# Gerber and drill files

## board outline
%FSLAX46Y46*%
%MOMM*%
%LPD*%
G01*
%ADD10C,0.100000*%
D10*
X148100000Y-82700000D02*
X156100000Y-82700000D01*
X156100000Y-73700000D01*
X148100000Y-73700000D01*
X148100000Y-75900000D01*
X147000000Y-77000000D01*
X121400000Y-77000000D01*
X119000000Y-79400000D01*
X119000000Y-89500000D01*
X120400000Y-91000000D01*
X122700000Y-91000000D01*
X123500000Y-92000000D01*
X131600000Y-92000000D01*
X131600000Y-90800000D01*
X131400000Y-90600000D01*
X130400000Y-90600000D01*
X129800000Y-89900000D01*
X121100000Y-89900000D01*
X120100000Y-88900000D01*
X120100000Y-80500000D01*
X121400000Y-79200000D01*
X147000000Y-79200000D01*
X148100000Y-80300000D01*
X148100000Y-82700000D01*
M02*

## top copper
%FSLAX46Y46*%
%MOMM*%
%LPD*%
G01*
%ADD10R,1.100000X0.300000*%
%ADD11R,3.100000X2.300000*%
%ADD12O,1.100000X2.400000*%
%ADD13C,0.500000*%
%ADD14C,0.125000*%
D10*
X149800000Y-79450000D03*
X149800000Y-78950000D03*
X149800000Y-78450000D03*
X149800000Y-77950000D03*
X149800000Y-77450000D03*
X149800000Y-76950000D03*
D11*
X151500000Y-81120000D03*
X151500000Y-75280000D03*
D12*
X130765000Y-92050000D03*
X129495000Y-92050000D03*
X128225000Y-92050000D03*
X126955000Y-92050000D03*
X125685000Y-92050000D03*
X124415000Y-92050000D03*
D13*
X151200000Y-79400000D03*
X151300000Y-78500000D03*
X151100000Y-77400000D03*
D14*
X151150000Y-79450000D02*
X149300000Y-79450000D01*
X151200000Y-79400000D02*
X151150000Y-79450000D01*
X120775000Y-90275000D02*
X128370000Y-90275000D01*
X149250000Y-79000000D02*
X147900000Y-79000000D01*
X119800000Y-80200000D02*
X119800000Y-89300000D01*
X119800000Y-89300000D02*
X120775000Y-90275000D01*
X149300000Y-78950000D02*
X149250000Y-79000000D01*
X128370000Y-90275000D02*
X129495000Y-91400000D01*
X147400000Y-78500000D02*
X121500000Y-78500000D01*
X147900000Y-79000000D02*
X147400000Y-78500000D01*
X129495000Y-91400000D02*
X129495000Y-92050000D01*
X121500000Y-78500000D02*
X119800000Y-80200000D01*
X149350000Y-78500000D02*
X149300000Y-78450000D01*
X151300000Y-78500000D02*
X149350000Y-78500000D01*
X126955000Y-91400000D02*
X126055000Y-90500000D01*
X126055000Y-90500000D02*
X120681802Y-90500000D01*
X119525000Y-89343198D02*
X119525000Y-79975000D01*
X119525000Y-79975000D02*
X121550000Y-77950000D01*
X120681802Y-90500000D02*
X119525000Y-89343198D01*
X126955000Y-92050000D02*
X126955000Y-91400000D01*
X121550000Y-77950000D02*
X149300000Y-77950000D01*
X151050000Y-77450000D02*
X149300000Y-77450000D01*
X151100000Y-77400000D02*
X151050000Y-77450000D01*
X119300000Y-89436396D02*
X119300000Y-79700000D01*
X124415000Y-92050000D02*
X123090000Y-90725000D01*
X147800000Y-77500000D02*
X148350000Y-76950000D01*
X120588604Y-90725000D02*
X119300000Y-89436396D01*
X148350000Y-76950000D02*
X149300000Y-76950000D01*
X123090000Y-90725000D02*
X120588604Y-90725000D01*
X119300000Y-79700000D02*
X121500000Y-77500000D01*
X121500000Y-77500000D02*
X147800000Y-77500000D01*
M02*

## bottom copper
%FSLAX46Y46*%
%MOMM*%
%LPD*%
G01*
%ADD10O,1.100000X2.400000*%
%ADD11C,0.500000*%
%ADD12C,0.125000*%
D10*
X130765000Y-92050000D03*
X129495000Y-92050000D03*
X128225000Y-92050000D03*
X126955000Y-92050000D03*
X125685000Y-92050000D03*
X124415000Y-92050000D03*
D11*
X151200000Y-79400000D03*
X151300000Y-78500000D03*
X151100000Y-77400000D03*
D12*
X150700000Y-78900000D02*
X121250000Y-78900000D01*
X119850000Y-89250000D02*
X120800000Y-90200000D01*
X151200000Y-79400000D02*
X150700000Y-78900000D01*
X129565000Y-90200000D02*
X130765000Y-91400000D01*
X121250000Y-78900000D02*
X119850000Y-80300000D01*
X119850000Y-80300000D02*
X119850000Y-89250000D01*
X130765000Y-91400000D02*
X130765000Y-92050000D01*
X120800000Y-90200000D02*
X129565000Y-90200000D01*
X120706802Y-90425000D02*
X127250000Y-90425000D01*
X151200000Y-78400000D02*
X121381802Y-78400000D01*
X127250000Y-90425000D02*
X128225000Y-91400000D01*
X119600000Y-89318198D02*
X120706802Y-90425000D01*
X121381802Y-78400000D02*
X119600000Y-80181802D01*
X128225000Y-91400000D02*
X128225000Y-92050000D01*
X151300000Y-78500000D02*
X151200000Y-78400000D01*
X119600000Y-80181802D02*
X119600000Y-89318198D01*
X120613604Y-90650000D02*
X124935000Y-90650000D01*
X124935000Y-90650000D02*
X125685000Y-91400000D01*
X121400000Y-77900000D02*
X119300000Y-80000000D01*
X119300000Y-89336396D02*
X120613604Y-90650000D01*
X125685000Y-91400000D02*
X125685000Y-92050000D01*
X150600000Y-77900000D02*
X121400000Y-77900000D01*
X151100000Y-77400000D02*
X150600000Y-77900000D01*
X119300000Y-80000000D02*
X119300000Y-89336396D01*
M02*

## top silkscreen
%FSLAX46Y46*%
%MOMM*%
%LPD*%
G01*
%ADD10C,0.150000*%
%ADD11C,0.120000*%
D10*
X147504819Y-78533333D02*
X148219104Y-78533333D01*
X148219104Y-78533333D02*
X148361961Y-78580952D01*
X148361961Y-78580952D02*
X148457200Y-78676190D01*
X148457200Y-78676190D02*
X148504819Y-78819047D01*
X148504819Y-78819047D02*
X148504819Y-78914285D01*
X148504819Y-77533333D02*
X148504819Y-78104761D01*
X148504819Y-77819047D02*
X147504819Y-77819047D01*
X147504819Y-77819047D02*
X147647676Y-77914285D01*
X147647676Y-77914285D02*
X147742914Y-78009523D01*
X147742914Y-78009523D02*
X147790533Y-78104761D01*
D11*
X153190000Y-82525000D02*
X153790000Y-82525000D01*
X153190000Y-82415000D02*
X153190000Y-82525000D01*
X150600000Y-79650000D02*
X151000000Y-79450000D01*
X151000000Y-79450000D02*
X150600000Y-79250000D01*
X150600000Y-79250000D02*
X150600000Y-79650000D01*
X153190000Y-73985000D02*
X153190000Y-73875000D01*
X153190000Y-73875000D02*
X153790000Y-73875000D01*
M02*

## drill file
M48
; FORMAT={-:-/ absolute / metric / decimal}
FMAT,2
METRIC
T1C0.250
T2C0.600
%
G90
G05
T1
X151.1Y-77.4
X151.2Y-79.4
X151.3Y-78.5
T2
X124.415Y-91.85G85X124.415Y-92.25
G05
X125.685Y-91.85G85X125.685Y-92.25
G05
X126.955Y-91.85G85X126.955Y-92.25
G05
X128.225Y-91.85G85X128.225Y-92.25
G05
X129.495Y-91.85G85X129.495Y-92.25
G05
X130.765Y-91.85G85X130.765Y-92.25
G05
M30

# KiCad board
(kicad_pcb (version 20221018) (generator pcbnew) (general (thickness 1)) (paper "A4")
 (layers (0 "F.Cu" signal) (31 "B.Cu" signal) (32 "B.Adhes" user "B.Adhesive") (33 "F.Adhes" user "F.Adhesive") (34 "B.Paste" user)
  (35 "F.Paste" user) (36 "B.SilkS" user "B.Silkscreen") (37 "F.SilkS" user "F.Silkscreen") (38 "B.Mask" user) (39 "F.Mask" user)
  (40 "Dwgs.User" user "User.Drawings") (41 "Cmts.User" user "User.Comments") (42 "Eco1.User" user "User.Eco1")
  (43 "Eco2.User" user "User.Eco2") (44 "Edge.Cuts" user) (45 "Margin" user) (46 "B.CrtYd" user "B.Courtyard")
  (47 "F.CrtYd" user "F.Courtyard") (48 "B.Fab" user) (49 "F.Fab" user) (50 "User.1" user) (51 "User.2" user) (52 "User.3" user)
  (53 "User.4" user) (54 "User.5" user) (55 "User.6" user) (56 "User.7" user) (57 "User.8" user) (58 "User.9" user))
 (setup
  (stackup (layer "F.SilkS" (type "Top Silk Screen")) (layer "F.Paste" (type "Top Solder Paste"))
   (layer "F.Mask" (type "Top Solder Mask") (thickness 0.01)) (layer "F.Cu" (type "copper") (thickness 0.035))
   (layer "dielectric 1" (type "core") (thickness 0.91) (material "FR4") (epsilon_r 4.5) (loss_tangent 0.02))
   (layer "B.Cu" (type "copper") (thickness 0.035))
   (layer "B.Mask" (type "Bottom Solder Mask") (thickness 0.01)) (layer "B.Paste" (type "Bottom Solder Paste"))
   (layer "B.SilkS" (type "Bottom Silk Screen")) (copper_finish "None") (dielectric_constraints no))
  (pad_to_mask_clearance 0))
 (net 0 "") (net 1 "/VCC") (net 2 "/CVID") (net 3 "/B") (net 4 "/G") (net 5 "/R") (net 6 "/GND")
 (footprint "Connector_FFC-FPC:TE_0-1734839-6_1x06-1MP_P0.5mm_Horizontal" (layer "F.Cu") (at 151.15 78.2 90)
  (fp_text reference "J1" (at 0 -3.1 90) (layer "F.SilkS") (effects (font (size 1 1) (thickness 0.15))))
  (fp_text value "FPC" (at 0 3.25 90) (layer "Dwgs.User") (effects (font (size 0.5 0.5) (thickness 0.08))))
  (fp_line (start -4.325 2.04) (end -4.325 2.64) (stroke (width 0.12) (type solid)) (layer "F.SilkS"))
  (fp_line (start -4.215 2.04) (end -4.325 2.04) (stroke (width 0.12) (type solid)) (layer "F.SilkS"))
  (fp_line (start -1.45 -0.55) (end -1.25 -0.15) (stroke (width 0.12) (type solid)) (layer "F.SilkS"))
  (fp_line (start -1.25 -0.15) (end -1.05 -0.55) (stroke (width 0.12) (type solid)) (layer "F.SilkS"))
  (fp_line (start -1.05 -0.55) (end -1.45 -0.55) (stroke (width 0.12) (type solid)) (layer "F.SilkS"))
  (fp_line (start 4.215 2.04) (end 4.325 2.04) (stroke (width 0.12) (type solid)) (layer "F.SilkS"))
  (fp_line (start 4.325 2.04) (end 4.325 2.64) (stroke (width 0.12) (type solid)) (layer "F.SilkS"))
  (pad "1" smd rect (at -1.25 -1.35 90) (size 0.3 1.1) (layers "F.Cu" "F.Paste" "F.Mask") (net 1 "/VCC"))
  (pad "2" smd rect (at -0.75 -1.35 90) (size 0.3 1.1) (layers "F.Cu" "F.Paste" "F.Mask") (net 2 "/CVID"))
  (pad "3" smd rect (at -0.25 -1.35 90) (size 0.3 1.1) (layers "F.Cu" "F.Paste" "F.Mask") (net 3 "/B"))
  (pad "4" smd rect (at 0.25 -1.35 90) (size 0.3 1.1) (layers "F.Cu" "F.Paste" "F.Mask") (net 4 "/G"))
  (pad "5" smd rect (at 0.75 -1.35 90) (size 0.3 1.1) (layers "F.Cu" "F.Paste" "F.Mask") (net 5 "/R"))
  (pad "6" smd rect (at 1.25 -1.35 90) (size 0.3 1.1) (layers "F.Cu" "F.Paste" "F.Mask") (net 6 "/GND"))
  (pad "MP" smd rect (at -2.92 0.35 90) (size 2.3 3.1) (layers "F.Cu" "F.Paste" "F.Mask"))
  (pad "MP" smd rect (at 2.92 0.35 90) (size 2.3 3.1) (layers "F.Cu" "F.Paste" "F.Mask")))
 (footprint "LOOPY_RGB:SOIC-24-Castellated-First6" (layer "F.Cu") (at 131.4 94.7)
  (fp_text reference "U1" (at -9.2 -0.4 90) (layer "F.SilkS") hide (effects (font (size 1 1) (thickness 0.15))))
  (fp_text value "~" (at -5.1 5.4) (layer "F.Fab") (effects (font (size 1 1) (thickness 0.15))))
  (pad "19" thru_hole oval (at -0.635 -2.65) (size 1.1 2.4) (drill oval 0.6 1) (layers "*.Cu" "*.Mask") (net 1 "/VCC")
   (thermal_bridge_angle 45))
  (pad "20" thru_hole oval (at -1.905 -2.65) (size 1.1 2.4) (drill oval 0.6 1) (layers "*.Cu" "*.Mask") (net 2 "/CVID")
   (thermal_bridge_angle 45))
  (pad "21" thru_hole oval (at -3.175 -2.65) (size 1.1 2.4) (drill oval 0.6 1) (layers "*.Cu" "*.Mask") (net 3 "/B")
   (thermal_bridge_angle 45))
  (pad "22" thru_hole oval (at -4.445 -2.65) (size 1.1 2.4) (drill oval 0.6 1) (layers "*.Cu" "*.Mask") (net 4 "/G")
   (thermal_bridge_angle 45))
  (pad "23" thru_hole oval (at -5.715 -2.65) (size 1.1 2.4) (drill oval 0.6 1) (layers "*.Cu" "*.Mask") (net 5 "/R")
   (thermal_bridge_angle 45))
  (pad "24" thru_hole oval (at -6.985 -2.65) (size 1.1 2.4) (drill oval 0.6 1) (layers "*.Cu" "*.Mask") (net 6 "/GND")
   (thermal_bridge_angle 45)))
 (gr_poly
  (pts (xy 148.1 82.7) (xy 156.1 82.7) (xy 156.1 73.7) (xy 148.1 73.7) (xy 148.1 75.9) (xy 147 77) (xy 121.4 77) (xy 119 79.4) (xy 119 89.5)
   (xy 120.4 91) (xy 122.7 91) (xy 123.5 92) (xy 131.6 92) (xy 131.6 90.8) (xy 131.4 90.6) (xy 130.4 90.6) (xy 129.8 89.9) (xy 121.1 89.9)
   (xy 120.1 88.9) (xy 120.1 80.5) (xy 121.4 79.2) (xy 147 79.2) (xy 148.1 80.3))
  (stroke (width 0.1) (type solid)) (fill none) (layer "Edge.Cuts"))
 (segment (start 151.15 79.45) (end 149.3 79.45) (width 0.125) (layer "F.Cu") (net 1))
 (segment (start 151.2 79.4) (end 151.15 79.45) (width 0.125) (layer "F.Cu") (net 1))
 (via (at 151.2 79.4) (size 0.5) (drill 0.25) (layers "F.Cu" "B.Cu") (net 1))
 (segment (start 150.7 78.9) (end 121.25 78.9) (width 0.125) (layer "B.Cu") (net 1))
 (segment (start 119.85 89.25) (end 120.8 90.2) (width 0.125) (layer "B.Cu") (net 1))
 (segment (start 151.2 79.4) (end 150.7 78.9) (width 0.125) (layer "B.Cu") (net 1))
 (segment (start 129.565 90.2) (end 130.765 91.4) (width 0.125) (layer "B.Cu") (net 1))
 (segment (start 121.25 78.9) (end 119.85 80.3) (width 0.125) (layer "B.Cu") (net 1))
 (segment (start 119.85 80.3) (end 119.85 89.25) (width 0.125) (layer "B.Cu") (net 1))
 (segment (start 130.765 91.4) (end 130.765 92.05) (width 0.125) (layer "B.Cu") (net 1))
 (segment (start 120.8 90.2) (end 129.565 90.2) (width 0.125) (layer "B.Cu") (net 1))
 (segment (start 120.775 90.275) (end 128.37 90.275) (width 0.125) (layer "F.Cu") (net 2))
 (segment (start 149.25 79) (end 147.9 79) (width 0.125) (layer "F.Cu") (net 2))
 (segment (start 119.8 80.2) (end 119.8 89.3) (width 0.125) (layer "F.Cu") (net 2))
 (segment (start 119.8 89.3) (end 120.775 90.275) (width 0.125) (layer "F.Cu") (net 2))
 (segment (start 149.3 78.95) (end 149.25 79) (width 0.125) (layer "F.Cu") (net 2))
 (segment (start 128.37 90.275) (end 129.495 91.4) (width 0.125) (layer "F.Cu") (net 2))
 (segment (start 147.4 78.5) (end 121.5 78.5) (width 0.125) (layer "F.Cu") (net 2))
 (segment (start 147.9 79) (end 147.4 78.5) (width 0.125) (layer "F.Cu") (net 2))
 (segment (start 129.495 91.4) (end 129.495 92.05) (width 0.125) (layer "F.Cu") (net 2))
 (segment (start 121.5 78.5) (end 119.8 80.2) (width 0.125) (layer "F.Cu") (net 2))
 (segment (start 149.35 78.5) (end 149.3 78.45) (width 0.125) (layer "F.Cu") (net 3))
 (segment (start 151.3 78.5) (end 149.35 78.5) (width 0.125) (layer "F.Cu") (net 3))
 (via (at 151.3 78.5) (size 0.5) (drill 0.25) (layers "F.Cu" "B.Cu") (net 3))
 (segment (start 120.706802 90.425) (end 127.25 90.425) (width 0.125) (layer "B.Cu") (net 3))
 (segment (start 151.2 78.4) (end 121.381802 78.4) (width 0.125) (layer "B.Cu") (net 3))
 (segment (start 127.25 90.425) (end 128.225 91.4) (width 0.125) (layer "B.Cu") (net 3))
 (segment (start 119.6 89.318198) (end 120.706802 90.425) (width 0.125) (layer "B.Cu") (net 3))
 (segment (start 121.381802 78.4) (end 119.6 80.181802) (width 0.125) (layer "B.Cu") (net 3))
 (segment (start 128.225 91.4) (end 128.225 92.05) (width 0.125) (layer "B.Cu") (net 3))
 (segment (start 151.3 78.5) (end 151.2 78.4) (width 0.125) (layer "B.Cu") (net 3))
 (segment (start 119.6 80.181802) (end 119.6 89.318198) (width 0.125) (layer "B.Cu") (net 3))
 (segment (start 126.955 91.4) (end 126.055 90.5) (width 0.125) (layer "F.Cu") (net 4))
 (segment (start 126.055 90.5) (end 120.681802 90.5) (width 0.125) (layer "F.Cu") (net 4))
 (segment (start 119.525 89.343198) (end 119.525 79.975) (width 0.125) (layer "F.Cu") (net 4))
 (segment (start 119.525 79.975) (end 121.55 77.95) (width 0.125) (layer "F.Cu") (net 4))
 (segment (start 120.681802 90.5) (end 119.525 89.343198) (width 0.125) (layer "F.Cu") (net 4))
 (segment (start 126.955 92.05) (end 126.955 91.4) (width 0.125) (layer "F.Cu") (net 4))
 (segment (start 121.55 77.95) (end 149.3 77.95) (width 0.125) (layer "F.Cu") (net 4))
 (segment (start 151.05 77.45) (end 149.3 77.45) (width 0.125) (layer "F.Cu") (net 5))
 (segment (start 151.1 77.4) (end 151.05 77.45) (width 0.125) (layer "F.Cu") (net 5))
 (via (at 151.1 77.4) (size 0.5) (drill 0.25) (layers "F.Cu" "B.Cu") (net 5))
 (segment (start 120.613604 90.65) (end 124.935 90.65) (width 0.125) (layer "B.Cu") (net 5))
 (segment (start 124.935 90.65) (end 125.685 91.4) (width 0.125) (layer "B.Cu") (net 5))
 (segment (start 121.4 77.9) (end 119.3 80) (width 0.125) (layer "B.Cu") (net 5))
 (segment (start 119.3 89.336396) (end 120.613604 90.65) (width 0.125) (layer "B.Cu") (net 5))
 (segment (start 125.685 91.4) (end 125.685 92.05) (width 0.125) (layer "B.Cu") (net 5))
 (segment (start 150.6 77.9) (end 121.4 77.9) (width 0.125) (layer "B.Cu") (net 5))
 (segment (start 151.1 77.4) (end 150.6 77.9) (width 0.125) (layer "B.Cu") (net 5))
 (segment (start 119.3 80) (end 119.3 89.336396) (width 0.125) (layer "B.Cu") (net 5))
 (segment (start 119.3 89.436396) (end 119.3 79.7) (width 0.125) (layer "F.Cu") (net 6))
 (segment (start 124.415 92.05) (end 123.09 90.725) (width 0.125) (layer "F.Cu") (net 6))
 (segment (start 147.8 77.5) (end 148.35 76.95) (width 0.125) (layer "F.Cu") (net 6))
 (segment (start 120.588604 90.725) (end 119.3 89.436396) (width 0.125) (layer "F.Cu") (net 6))
 (segment (start 148.35 76.95) (end 149.3 76.95) (width 0.125) (layer "F.Cu") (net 6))
 (segment (start 123.09 90.725) (end 120.588604 90.725) (width 0.125) (layer "F.Cu") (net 6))
 (segment (start 119.3 79.7) (end 121.5 77.5) (width 0.125) (layer "F.Cu") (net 6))
 (segment (start 121.5 77.5) (end 147.8 77.5) (width 0.125) (layer "F.Cu") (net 6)))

